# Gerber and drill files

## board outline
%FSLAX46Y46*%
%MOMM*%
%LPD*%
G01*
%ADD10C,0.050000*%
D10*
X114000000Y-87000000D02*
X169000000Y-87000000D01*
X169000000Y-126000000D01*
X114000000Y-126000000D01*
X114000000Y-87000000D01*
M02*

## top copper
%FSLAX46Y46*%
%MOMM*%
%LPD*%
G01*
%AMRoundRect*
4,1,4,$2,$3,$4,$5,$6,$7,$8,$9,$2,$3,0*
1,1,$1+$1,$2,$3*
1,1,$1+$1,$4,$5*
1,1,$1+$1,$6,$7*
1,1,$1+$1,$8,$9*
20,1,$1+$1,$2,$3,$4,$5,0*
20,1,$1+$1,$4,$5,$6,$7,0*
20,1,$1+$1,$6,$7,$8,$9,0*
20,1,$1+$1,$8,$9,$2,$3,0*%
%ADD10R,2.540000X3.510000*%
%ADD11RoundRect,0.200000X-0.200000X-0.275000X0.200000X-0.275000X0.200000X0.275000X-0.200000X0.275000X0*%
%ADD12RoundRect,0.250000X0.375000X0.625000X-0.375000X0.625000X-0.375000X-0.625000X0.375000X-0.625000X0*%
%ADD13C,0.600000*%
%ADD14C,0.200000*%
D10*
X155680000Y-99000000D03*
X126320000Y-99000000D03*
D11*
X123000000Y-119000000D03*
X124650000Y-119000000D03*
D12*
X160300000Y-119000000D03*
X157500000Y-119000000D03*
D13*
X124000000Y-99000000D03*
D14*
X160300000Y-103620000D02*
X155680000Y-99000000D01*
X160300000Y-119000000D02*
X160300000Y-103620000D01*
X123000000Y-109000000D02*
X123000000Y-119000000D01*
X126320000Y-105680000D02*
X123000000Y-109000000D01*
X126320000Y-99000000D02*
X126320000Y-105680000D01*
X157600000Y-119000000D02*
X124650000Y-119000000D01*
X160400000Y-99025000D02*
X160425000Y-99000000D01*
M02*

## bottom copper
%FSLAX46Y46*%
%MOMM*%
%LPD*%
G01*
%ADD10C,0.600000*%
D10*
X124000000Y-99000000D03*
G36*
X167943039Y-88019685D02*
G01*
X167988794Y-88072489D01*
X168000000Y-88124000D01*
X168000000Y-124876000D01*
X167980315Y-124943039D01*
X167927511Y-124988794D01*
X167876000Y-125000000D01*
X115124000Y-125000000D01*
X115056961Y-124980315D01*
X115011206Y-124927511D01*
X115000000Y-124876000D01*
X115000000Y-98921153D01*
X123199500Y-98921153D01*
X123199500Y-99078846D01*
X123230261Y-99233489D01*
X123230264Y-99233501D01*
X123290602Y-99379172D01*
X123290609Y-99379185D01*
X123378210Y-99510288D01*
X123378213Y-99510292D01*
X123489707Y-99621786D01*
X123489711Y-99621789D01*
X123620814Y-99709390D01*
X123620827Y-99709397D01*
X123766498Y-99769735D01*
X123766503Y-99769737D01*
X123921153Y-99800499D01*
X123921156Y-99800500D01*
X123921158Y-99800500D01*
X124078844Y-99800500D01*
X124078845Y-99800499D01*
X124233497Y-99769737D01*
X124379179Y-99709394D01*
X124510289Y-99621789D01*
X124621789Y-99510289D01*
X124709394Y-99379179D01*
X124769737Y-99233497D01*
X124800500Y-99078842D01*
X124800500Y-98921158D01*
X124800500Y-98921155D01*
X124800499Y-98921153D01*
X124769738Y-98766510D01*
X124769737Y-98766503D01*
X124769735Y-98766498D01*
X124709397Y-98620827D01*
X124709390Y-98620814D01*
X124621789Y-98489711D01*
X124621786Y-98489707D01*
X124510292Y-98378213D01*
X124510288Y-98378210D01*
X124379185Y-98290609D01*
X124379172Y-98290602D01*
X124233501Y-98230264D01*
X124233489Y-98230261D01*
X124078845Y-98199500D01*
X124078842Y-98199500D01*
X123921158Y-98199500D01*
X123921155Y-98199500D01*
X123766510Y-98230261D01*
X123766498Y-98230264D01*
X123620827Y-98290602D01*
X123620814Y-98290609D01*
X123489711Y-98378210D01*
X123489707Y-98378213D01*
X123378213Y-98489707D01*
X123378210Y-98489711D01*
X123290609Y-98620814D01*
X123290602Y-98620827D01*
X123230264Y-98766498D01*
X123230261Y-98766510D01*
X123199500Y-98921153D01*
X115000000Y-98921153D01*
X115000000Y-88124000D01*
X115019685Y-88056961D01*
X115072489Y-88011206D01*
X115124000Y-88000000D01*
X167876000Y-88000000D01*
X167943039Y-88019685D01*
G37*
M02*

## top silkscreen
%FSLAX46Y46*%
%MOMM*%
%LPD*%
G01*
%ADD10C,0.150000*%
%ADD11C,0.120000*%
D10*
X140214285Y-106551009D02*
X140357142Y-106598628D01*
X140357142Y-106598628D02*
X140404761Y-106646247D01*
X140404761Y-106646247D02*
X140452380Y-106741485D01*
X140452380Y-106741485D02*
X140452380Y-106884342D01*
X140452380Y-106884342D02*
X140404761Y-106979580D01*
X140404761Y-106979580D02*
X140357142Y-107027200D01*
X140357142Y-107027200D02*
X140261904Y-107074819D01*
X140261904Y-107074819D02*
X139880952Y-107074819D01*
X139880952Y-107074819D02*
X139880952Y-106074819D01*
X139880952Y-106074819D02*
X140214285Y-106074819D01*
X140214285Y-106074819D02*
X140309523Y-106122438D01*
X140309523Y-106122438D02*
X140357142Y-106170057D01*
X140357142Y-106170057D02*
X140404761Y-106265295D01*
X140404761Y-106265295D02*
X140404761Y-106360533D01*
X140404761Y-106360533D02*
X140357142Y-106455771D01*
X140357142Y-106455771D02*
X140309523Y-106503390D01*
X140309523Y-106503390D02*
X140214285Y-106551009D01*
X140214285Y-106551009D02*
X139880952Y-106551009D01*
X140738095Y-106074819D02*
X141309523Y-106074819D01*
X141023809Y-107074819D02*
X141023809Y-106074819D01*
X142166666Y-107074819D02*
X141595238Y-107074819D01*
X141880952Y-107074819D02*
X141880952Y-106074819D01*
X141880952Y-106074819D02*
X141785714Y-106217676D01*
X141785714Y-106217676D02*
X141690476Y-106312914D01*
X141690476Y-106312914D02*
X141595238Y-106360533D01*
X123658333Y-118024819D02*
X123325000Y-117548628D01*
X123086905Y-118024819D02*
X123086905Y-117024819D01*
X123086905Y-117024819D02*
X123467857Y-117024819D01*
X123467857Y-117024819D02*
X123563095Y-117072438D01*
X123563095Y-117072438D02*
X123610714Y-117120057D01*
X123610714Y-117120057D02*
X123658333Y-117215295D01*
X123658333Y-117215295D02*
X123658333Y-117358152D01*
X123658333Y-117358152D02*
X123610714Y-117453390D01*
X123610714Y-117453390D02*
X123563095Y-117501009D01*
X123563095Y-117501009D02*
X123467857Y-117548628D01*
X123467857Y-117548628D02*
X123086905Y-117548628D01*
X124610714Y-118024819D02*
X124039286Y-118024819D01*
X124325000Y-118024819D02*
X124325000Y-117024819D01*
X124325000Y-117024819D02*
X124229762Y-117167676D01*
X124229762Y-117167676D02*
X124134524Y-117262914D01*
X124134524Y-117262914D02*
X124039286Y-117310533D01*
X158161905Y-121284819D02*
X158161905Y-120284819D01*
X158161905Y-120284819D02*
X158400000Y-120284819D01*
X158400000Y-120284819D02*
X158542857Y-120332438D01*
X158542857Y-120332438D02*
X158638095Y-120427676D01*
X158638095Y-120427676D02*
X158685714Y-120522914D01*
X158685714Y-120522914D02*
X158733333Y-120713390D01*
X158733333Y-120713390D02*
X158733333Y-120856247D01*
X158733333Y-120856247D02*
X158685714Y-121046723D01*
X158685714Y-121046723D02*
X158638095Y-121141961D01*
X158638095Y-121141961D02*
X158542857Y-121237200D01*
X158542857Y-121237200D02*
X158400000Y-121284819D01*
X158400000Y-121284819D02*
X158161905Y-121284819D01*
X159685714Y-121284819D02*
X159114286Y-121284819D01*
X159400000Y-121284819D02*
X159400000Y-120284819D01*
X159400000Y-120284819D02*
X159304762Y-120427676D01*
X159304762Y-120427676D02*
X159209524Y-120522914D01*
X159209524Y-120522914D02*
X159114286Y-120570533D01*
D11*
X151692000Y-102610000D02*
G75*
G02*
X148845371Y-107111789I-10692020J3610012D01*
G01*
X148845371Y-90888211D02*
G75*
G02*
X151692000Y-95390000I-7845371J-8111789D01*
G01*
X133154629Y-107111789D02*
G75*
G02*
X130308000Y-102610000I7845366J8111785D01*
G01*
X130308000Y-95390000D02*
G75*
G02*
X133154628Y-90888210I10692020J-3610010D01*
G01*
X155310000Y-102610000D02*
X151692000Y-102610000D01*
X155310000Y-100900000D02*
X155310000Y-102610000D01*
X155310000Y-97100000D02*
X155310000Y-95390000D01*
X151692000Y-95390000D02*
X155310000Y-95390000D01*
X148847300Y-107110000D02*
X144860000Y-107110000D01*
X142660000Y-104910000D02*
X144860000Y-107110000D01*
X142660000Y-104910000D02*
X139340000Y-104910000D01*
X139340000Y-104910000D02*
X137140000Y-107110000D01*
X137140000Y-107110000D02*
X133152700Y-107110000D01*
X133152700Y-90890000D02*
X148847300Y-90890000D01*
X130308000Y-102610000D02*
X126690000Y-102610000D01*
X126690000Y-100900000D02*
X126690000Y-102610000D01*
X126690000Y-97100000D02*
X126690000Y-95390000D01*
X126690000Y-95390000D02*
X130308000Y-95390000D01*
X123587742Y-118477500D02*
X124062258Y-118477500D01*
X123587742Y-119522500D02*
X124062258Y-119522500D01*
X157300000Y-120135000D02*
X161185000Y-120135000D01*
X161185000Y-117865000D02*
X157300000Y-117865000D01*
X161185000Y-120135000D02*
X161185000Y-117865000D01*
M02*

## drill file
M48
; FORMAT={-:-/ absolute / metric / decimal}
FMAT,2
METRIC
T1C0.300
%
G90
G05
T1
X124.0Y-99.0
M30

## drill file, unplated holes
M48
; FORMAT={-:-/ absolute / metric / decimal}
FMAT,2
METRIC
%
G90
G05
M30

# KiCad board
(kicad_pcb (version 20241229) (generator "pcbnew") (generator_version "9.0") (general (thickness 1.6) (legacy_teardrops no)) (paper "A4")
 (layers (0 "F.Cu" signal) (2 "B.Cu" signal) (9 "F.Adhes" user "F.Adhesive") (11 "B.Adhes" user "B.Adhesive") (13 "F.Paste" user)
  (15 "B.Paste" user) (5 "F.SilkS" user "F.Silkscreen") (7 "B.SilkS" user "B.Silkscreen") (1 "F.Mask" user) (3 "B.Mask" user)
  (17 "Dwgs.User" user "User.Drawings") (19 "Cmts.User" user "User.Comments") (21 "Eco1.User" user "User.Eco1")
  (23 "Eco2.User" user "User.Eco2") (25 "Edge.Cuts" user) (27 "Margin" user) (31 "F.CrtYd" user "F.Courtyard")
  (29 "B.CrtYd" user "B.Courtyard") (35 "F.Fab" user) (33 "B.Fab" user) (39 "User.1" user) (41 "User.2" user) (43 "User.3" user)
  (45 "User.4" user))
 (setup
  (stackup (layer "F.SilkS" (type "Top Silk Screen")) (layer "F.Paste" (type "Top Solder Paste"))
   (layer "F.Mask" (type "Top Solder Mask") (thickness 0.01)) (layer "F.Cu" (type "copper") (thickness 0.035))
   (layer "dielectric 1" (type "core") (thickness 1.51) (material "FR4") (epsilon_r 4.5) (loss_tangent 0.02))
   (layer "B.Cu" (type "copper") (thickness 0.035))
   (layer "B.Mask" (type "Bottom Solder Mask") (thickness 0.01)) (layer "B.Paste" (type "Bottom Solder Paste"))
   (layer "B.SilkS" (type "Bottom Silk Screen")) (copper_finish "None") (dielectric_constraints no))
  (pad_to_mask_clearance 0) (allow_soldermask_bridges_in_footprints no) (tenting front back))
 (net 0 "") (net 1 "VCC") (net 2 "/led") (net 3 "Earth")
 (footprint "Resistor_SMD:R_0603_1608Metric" (layer "F.Cu") (at 123.825 119)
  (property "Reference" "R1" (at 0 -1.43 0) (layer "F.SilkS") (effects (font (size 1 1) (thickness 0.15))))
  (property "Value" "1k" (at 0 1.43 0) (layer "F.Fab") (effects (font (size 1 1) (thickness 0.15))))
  (fp_line (start -0.237258 -0.5225) (end 0.237258 -0.5225) (stroke (width 0.12) (type solid)) (layer "F.SilkS"))
  (fp_line (start -0.237258 0.5225) (end 0.237258 0.5225) (stroke (width 0.12) (type solid)) (layer "F.SilkS"))
  (pad "1" smd roundrect (at -0.825 0) (size 0.8 0.95) (layers "F.Cu" "F.Mask" "F.Paste") (roundrect_rratio 0.25) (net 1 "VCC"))
  (pad "2" smd roundrect (at 0.825 0) (size 0.8 0.95) (layers "F.Cu" "F.Mask" "F.Paste") (roundrect_rratio 0.25) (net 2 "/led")))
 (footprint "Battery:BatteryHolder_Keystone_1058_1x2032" (layer "F.Cu") (at 141 99)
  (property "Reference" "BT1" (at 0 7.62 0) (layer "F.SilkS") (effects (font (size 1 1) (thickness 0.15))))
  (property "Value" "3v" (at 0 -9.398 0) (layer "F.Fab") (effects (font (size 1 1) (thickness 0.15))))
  (fp_line (start -14.31 -3.61) (end -10.692 -3.61) (stroke (width 0.12) (type solid)) (layer "F.SilkS"))
  (fp_line (start -14.31 -1.9) (end -14.31 -3.61) (stroke (width 0.12) (type solid)) (layer "F.SilkS"))
  (fp_line (start -14.31 1.9) (end -14.31 3.61) (stroke (width 0.12) (type solid)) (layer "F.SilkS"))
  (fp_line (start -10.692 3.61) (end -14.31 3.61) (stroke (width 0.12) (type solid)) (layer "F.SilkS"))
  (fp_line (start -7.8473 -8.11) (end 7.8473 -8.11) (stroke (width 0.12) (type solid)) (layer "F.SilkS"))
  (fp_line (start -3.86 8.11) (end -7.8473 8.11) (stroke (width 0.12) (type solid)) (layer "F.SilkS"))
  (fp_line (start -1.66 5.91) (end -3.86 8.11) (stroke (width 0.12) (type solid)) (layer "F.SilkS"))
  (fp_line (start 1.66 5.91) (end -1.66 5.91) (stroke (width 0.12) (type solid)) (layer "F.SilkS"))
  (fp_line (start 1.66 5.91) (end 3.86 8.11) (stroke (width 0.12) (type solid)) (layer "F.SilkS"))
  (fp_line (start 7.8473 8.11) (end 3.86 8.11) (stroke (width 0.12) (type solid)) (layer "F.SilkS"))
  (fp_line (start 10.692 -3.61) (end 14.31 -3.61) (stroke (width 0.12) (type solid)) (layer "F.SilkS"))
  (fp_line (start 14.31 -1.9) (end 14.31 -3.61) (stroke (width 0.12) (type solid)) (layer "F.SilkS"))
  (fp_line (start 14.31 1.9) (end 14.31 3.61) (stroke (width 0.12) (type solid)) (layer "F.SilkS"))
  (fp_line (start 14.31 3.61) (end 10.692 3.61) (stroke (width 0.12) (type solid)) (layer "F.SilkS"))
  (fp_arc (start -10.692 -3.61) (mid -9.538084 -6.031244) (end -7.845371 -8.111789) (stroke (width 0.12) (type solid)) (layer "F.SilkS"))
  (fp_arc (start -7.845371 8.111789) (mid -9.538085 6.031244) (end -10.692 3.61) (stroke (width 0.12) (type solid)) (layer "F.SilkS"))
  (fp_arc (start 7.845371 -8.111789) (mid 9.538085 -6.031244) (end 10.692 -3.61) (stroke (width 0.12) (type solid)) (layer "F.SilkS"))
  (fp_arc (start 10.692 3.61) (mid 9.538084 6.031244) (end 7.845371 8.111789) (stroke (width 0.12) (type solid)) (layer "F.SilkS"))
  (pad "1" smd rect (at -14.68 0) (size 2.54 3.51) (layers "F.Cu" "F.Mask" "F.Paste") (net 1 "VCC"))
  (pad "2" smd rect (at 14.68 0) (size 2.54 3.51) (layers "F.Cu" "F.Mask" "F.Paste") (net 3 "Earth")))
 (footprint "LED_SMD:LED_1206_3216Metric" (layer "F.Cu") (at 158.9 119 180)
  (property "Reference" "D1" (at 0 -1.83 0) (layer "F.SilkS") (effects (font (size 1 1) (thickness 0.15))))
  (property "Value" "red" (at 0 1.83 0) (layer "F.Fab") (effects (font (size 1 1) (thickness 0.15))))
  (fp_line (start 1.6 -1.135) (end -2.285 -1.135) (stroke (width 0.12) (type solid)) (layer "F.SilkS"))
  (fp_line (start -2.285 1.135) (end 1.6 1.135) (stroke (width 0.12) (type solid)) (layer "F.SilkS"))
  (fp_line (start -2.285 -1.135) (end -2.285 1.135) (stroke (width 0.12) (type solid)) (layer "F.SilkS"))
  (pad "1" smd roundrect (at -1.4 0 180) (size 1.25 1.75) (layers "F.Cu" "F.Mask" "F.Paste") (roundrect_rratio 0.2) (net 3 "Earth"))
  (pad "2" smd roundrect (at 1.4 0 180) (size 1.25 1.75) (layers "F.Cu" "F.Mask" "F.Paste") (roundrect_rratio 0.2) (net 2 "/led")))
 (gr_rect (start 114 87) (end 169 126) (stroke (width 0.05) (type default)) (fill no) (layer "Edge.Cuts"))
 (segment (start 126.32 105.68) (end 123 109) (width 0.2) (layer "F.Cu") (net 1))
 (segment (start 126.32 99) (end 126.32 105.68) (width 0.2) (layer "F.Cu") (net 1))
 (segment (start 123 109) (end 123 119) (width 0.2) (layer "F.Cu") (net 1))
 (via (at 124 99) (size 0.6) (drill 0.3) (layers "F.Cu" "B.Cu") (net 1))
 (segment (start 160.3 119) (end 160.3 103.62) (width 0.2) (layer "F.Cu") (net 3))
 (segment (start 160.3 103.62) (end 155.68 99) (width 0.2) (layer "F.Cu") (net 3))
 (segment (start 160.4 99.025) (end 160.425 99) (width 0.2) (layer "F.Cu") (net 3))
 (segment (start 157.6 119) (end 124.65 119) (width 0.2) (layer "F.Cu") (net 2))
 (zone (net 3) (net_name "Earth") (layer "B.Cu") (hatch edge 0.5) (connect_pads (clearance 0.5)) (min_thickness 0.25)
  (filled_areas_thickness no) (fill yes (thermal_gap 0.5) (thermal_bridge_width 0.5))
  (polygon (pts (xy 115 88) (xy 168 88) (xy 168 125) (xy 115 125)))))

